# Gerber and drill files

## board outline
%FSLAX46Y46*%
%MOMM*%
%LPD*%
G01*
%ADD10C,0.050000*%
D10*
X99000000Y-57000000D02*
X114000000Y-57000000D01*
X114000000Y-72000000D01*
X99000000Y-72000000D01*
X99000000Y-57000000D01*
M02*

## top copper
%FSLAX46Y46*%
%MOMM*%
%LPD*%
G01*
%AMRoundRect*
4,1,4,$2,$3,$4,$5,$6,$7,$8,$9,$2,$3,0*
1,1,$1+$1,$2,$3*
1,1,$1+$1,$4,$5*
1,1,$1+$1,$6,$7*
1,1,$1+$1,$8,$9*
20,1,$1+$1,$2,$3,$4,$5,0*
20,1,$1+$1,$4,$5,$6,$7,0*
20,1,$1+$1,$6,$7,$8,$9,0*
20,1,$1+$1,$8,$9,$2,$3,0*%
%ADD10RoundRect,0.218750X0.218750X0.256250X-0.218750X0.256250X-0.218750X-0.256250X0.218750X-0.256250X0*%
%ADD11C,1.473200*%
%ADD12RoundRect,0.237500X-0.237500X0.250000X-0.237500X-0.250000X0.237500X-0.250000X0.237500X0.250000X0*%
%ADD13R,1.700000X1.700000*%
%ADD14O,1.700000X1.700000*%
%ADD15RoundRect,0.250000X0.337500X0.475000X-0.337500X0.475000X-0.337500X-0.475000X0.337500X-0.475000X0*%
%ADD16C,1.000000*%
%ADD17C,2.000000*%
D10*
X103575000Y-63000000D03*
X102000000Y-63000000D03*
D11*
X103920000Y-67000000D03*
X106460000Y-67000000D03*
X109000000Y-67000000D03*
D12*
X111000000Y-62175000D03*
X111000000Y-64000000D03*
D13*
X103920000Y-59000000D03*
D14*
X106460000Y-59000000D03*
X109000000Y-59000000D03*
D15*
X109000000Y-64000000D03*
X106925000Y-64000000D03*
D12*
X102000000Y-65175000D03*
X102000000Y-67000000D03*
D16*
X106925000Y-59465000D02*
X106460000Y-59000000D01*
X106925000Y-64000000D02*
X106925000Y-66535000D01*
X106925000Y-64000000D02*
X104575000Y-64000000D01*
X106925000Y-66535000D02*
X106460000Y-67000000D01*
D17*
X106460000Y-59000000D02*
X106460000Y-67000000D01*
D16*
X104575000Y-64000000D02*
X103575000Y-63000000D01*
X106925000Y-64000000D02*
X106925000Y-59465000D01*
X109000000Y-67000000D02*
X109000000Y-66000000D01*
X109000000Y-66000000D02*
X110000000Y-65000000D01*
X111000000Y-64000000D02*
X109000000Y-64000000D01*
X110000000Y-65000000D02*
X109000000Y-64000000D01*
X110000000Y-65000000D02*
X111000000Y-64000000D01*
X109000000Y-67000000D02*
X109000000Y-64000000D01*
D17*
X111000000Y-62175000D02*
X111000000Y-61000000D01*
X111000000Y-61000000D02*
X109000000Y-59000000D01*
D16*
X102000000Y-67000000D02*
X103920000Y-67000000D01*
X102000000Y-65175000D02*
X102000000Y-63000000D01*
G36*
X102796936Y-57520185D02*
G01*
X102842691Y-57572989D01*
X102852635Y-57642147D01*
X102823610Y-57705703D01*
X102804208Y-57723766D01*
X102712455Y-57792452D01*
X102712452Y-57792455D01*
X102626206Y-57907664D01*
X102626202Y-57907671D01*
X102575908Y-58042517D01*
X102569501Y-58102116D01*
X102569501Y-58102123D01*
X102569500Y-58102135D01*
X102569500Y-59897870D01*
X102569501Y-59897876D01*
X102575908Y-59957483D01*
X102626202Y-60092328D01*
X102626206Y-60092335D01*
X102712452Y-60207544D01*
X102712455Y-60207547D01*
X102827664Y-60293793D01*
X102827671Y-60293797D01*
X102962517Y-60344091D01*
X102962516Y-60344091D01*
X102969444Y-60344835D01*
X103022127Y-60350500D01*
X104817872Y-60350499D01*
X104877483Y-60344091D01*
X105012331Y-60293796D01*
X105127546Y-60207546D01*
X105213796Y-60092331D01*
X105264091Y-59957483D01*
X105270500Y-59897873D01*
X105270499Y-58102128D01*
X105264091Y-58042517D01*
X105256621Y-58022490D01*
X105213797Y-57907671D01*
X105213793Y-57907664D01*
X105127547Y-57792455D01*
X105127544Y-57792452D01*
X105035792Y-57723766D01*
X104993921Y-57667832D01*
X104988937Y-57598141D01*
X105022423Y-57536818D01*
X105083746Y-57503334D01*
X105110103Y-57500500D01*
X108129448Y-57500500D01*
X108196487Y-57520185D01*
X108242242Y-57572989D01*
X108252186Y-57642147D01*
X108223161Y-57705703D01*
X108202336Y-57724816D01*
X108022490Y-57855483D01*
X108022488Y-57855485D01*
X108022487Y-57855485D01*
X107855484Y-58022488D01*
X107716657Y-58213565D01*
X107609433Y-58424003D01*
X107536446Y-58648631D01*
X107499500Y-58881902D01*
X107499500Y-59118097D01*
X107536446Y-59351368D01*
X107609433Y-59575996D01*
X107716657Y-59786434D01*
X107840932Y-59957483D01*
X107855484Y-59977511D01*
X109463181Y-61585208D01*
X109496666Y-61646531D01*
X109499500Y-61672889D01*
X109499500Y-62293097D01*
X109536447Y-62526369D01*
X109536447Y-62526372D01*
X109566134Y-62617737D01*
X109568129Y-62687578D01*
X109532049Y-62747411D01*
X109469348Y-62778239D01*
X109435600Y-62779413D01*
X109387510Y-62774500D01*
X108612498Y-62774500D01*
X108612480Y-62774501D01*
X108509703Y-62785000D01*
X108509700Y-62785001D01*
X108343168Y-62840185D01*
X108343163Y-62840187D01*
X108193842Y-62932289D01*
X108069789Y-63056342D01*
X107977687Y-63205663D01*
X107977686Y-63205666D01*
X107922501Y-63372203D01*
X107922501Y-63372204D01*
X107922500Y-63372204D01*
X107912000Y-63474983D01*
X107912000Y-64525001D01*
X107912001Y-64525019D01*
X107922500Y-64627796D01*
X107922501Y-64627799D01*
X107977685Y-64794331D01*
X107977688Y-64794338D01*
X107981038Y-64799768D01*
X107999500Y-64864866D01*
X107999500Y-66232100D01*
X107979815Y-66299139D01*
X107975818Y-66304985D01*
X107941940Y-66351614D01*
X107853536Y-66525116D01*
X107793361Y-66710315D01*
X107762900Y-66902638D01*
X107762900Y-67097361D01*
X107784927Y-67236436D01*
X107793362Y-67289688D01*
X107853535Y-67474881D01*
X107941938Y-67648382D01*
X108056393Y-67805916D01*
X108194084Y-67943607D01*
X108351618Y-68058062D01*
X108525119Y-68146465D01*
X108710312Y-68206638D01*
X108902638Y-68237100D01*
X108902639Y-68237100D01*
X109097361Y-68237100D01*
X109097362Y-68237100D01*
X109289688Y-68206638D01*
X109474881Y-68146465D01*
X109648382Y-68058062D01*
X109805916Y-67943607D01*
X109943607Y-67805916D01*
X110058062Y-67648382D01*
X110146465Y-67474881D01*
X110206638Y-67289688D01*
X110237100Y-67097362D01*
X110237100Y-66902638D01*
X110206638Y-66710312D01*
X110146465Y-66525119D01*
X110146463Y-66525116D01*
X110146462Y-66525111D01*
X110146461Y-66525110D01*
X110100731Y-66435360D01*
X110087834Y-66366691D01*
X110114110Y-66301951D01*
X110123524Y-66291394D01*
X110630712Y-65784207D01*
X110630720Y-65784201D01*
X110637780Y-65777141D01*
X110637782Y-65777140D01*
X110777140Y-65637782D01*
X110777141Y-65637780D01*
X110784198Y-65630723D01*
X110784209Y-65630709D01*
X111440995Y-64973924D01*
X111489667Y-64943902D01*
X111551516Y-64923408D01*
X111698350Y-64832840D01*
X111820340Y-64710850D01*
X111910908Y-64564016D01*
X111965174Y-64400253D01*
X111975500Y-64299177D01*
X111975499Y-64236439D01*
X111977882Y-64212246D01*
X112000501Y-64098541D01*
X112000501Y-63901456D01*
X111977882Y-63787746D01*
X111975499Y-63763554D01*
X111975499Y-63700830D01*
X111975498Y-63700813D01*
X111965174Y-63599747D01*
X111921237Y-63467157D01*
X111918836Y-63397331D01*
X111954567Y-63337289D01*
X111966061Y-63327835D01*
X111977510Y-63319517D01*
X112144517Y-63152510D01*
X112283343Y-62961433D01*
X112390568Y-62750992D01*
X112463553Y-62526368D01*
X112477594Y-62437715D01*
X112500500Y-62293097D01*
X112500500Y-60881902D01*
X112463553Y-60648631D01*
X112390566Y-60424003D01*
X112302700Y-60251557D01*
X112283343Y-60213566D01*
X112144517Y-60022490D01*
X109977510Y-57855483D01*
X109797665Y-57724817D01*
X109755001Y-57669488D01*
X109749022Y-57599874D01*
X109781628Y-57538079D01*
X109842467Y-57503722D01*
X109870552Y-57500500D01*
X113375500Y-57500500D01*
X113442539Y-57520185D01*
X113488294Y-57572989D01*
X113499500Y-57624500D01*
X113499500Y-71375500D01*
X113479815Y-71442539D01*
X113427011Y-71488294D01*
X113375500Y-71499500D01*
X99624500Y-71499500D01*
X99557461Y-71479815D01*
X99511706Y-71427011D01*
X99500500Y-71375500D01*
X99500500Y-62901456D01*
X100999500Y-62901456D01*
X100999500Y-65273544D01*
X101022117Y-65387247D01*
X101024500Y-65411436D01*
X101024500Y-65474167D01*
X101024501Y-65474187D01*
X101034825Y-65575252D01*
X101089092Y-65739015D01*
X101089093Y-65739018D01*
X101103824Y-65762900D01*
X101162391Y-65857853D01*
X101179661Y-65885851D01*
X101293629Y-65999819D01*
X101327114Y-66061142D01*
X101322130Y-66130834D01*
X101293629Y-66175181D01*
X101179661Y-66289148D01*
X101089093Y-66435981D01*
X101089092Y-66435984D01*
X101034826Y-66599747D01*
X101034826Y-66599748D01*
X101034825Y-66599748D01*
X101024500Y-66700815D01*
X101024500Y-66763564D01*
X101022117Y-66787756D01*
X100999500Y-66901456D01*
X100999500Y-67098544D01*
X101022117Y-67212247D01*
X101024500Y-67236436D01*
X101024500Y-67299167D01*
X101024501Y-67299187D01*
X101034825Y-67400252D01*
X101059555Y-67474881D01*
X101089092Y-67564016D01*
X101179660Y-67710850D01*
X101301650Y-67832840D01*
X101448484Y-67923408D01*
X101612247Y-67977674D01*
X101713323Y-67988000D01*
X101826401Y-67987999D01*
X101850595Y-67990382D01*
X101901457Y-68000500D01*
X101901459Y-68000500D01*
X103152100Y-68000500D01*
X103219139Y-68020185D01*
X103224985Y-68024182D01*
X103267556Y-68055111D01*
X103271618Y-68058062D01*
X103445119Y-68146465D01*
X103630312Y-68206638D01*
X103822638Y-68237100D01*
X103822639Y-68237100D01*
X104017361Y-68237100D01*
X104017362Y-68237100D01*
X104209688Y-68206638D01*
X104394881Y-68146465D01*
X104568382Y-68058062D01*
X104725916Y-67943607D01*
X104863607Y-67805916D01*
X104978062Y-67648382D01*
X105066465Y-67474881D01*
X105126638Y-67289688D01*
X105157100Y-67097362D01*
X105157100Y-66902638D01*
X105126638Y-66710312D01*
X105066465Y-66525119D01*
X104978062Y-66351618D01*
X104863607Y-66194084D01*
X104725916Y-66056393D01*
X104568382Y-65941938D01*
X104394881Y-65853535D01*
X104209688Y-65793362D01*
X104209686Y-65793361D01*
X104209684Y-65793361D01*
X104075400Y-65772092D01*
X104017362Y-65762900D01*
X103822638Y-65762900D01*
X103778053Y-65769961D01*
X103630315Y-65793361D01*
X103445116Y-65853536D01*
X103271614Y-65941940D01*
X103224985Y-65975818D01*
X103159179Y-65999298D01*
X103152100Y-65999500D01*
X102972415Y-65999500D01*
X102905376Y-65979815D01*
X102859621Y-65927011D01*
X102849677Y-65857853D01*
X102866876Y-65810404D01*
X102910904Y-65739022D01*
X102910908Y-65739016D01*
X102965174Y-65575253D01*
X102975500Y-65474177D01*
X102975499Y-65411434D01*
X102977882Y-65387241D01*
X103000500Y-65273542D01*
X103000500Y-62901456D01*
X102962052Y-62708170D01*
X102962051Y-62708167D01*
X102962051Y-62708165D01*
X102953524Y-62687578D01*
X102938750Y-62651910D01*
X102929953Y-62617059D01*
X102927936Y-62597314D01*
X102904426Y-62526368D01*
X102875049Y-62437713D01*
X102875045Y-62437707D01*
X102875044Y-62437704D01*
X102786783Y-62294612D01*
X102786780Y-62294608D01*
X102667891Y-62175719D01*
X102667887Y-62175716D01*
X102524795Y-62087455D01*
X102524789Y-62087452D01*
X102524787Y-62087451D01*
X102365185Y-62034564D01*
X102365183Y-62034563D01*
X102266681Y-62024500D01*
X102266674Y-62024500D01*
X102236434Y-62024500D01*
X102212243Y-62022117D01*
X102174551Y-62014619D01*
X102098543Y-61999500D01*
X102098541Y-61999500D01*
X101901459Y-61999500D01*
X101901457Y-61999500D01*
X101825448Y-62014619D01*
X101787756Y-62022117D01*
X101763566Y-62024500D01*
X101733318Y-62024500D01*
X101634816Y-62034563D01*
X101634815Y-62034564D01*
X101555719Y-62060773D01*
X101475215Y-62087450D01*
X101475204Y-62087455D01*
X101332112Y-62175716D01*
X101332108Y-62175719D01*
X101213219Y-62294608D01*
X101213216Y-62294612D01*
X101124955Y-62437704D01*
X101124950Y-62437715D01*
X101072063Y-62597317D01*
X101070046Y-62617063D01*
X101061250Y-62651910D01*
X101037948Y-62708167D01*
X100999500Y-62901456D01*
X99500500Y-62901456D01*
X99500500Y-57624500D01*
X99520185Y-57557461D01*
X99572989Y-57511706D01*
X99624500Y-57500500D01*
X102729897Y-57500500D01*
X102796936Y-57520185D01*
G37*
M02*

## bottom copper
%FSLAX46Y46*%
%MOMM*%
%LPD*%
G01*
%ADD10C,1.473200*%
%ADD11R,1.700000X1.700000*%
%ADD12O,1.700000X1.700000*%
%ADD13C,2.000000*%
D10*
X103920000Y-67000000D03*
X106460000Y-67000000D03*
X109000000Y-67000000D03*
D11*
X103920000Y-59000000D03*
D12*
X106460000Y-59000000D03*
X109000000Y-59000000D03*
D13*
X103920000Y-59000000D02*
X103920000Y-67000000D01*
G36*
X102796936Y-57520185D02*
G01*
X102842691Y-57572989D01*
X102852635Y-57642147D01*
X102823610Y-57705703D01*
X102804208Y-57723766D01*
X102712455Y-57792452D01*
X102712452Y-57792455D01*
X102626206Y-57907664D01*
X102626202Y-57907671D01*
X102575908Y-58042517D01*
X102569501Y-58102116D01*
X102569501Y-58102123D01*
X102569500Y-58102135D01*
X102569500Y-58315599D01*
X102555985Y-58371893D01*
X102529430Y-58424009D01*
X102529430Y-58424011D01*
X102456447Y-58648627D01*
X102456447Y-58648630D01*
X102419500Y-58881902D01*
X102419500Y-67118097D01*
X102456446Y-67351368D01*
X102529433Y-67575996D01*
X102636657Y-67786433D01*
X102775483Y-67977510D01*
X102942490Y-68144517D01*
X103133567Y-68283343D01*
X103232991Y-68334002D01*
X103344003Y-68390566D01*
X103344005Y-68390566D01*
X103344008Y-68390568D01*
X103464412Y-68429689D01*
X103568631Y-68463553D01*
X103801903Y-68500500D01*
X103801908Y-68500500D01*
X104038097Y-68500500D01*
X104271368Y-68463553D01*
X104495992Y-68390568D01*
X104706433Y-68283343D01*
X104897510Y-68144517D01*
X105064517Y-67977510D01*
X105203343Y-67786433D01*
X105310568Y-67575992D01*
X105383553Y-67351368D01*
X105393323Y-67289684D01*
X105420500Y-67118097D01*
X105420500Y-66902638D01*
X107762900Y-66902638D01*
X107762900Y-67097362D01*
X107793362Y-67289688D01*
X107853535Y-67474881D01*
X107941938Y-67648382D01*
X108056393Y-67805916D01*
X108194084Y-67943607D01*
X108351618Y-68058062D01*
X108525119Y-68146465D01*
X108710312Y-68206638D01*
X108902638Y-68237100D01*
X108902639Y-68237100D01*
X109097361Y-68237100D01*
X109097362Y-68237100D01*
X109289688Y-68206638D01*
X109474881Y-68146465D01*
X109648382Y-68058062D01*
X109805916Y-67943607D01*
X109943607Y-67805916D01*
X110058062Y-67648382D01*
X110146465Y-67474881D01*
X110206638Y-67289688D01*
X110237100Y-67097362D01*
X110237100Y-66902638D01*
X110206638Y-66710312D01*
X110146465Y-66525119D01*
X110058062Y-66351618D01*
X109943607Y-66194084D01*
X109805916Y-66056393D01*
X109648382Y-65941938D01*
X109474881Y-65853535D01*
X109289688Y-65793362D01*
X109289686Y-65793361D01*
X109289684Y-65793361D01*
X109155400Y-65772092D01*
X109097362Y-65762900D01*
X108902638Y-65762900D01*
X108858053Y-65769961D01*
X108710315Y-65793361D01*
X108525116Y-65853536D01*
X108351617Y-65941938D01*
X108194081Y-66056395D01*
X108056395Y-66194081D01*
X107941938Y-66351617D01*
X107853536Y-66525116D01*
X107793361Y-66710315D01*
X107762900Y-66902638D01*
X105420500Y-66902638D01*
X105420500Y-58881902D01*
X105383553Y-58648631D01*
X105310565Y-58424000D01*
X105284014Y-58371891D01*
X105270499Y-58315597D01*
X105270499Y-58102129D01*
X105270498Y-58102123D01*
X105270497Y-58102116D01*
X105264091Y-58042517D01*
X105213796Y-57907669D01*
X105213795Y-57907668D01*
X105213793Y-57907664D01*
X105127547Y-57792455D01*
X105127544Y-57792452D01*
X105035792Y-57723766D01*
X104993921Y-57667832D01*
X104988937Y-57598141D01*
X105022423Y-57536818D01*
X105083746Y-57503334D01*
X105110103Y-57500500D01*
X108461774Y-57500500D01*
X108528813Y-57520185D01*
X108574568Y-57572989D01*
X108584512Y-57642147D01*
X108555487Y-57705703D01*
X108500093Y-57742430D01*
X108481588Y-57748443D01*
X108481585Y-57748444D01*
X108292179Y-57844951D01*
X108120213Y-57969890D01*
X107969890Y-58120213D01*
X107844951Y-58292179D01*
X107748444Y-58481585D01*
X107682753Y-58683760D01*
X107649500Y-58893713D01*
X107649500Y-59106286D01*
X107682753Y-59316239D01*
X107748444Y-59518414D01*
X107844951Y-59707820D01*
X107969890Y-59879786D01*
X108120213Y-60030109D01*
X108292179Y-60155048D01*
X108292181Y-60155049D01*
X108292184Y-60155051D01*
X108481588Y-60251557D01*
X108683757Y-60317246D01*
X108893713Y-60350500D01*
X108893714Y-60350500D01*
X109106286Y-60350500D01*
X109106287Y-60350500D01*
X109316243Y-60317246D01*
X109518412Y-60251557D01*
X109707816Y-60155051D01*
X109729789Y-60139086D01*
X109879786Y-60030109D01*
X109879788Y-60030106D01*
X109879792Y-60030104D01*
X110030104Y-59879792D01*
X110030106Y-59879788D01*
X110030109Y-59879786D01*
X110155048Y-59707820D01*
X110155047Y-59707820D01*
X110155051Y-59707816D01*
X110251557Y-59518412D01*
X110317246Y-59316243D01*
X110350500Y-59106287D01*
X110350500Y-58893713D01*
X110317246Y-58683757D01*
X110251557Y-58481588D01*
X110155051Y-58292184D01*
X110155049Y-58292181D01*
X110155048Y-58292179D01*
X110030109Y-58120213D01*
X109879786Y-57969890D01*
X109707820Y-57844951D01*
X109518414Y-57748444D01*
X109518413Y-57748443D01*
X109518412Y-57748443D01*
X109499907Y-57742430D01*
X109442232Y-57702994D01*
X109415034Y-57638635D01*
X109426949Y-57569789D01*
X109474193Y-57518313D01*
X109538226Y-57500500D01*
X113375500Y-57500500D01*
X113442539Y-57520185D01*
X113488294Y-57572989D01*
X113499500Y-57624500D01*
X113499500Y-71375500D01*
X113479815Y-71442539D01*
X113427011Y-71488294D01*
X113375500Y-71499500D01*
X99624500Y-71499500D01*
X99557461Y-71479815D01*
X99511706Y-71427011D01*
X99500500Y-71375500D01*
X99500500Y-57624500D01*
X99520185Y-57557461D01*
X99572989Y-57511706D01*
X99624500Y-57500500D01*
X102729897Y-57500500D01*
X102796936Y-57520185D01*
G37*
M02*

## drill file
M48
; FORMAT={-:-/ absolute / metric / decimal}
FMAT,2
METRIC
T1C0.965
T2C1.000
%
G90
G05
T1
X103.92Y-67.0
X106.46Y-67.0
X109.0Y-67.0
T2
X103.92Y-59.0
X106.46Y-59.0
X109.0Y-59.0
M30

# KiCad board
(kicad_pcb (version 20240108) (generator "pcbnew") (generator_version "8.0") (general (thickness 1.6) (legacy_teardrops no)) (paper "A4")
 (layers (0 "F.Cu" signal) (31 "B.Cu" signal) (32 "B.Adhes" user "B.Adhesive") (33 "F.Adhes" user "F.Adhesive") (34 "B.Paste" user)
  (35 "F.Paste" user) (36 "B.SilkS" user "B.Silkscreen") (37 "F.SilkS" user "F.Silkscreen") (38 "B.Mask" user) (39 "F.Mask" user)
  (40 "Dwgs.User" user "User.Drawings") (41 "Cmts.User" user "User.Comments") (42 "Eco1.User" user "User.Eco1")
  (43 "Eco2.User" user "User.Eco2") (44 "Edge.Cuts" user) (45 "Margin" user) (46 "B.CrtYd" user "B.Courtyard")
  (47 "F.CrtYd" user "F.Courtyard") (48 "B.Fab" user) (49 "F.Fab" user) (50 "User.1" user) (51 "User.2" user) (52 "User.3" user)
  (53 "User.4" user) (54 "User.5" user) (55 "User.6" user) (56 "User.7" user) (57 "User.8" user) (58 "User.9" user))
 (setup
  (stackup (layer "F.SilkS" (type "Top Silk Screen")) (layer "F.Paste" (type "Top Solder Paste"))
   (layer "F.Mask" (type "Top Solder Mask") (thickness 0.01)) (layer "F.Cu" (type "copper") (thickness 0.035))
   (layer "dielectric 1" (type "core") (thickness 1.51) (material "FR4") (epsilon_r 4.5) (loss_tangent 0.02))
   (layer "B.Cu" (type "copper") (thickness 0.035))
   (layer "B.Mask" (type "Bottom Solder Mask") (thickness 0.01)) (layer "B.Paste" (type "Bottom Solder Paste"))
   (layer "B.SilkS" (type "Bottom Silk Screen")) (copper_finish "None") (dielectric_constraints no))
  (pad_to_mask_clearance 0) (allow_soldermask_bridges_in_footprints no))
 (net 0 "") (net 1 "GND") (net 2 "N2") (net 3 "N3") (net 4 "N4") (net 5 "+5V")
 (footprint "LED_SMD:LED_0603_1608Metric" (layer "F.Cu") (at 102.7875 63 180)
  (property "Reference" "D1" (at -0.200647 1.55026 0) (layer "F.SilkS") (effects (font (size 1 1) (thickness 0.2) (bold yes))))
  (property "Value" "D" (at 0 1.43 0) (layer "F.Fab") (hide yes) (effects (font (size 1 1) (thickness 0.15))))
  (pad "1" smd roundrect (at -0.7875 0 180) (size 0.875 0.95) (layers "F.Cu" "F.Paste" "F.Mask") (roundrect_rratio 0.25) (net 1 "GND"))
  (pad "2" smd roundrect (at 0.7875 0 180) (size 0.875 0.95) (layers "F.Cu" "F.Paste" "F.Mask") (roundrect_rratio 0.25) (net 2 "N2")))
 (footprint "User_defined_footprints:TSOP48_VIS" (layer "F.Cu") (at 103.927304 66.99058)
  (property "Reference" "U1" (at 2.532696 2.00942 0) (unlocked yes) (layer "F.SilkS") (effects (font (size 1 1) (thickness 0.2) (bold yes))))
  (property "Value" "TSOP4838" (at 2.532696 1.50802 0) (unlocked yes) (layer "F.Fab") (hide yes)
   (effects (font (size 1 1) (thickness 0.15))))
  (pad "1" thru_hole circle (at -0.007304 0.00942) (size 1.4732 1.4732) (drill 0.9652) (layers "*.Cu" "*.Mask") (remove_unused_layers no)
   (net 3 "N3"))
  (pad "2" thru_hole circle (at 2.532696 0.00942) (size 1.4732 1.4732) (drill 0.9652) (layers "*.Cu" "*.Mask") (remove_unused_layers no)
   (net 1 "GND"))
  (pad "3" thru_hole circle (at 5.072696 0.00942) (size 1.4732 1.4732) (drill 0.9652) (layers "*.Cu" "*.Mask") (remove_unused_layers no)
   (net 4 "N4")))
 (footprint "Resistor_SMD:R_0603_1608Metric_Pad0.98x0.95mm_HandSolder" (layer "F.Cu") (at 111 63.0875 -90)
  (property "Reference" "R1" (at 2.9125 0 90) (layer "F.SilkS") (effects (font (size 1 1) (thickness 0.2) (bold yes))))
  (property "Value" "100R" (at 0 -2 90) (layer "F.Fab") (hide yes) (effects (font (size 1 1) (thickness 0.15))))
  (pad "1" smd roundrect (at -0.9125 0 270) (size 0.975 0.95) (layers "F.Cu" "F.Paste" "F.Mask") (roundrect_rratio 0.25) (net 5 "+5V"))
  (pad "2" smd roundrect (at 0.9125 0 270) (size 0.975 0.95) (layers "F.Cu" "F.Paste" "F.Mask") (roundrect_rratio 0.25) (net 4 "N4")))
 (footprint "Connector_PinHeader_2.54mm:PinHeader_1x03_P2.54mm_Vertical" (layer "F.Cu") (at 103.92 59 90)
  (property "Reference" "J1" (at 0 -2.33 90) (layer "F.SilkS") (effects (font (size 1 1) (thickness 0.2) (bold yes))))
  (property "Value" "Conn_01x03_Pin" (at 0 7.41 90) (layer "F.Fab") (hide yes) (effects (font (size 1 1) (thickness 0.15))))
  (pad "1" thru_hole rect (at 0 0 90) (size 1.7 1.7) (drill 1) (layers "*.Cu" "*.Mask") (remove_unused_layers no) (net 3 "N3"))
  (pad "2" thru_hole oval (at 0 2.54 90) (size 1.7 1.7) (drill 1) (layers "*.Cu" "*.Mask") (remove_unused_layers no) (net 1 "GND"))
  (pad "3" thru_hole oval (at 0 5.08 90) (size 1.7 1.7) (drill 1) (layers "*.Cu" "*.Mask") (remove_unused_layers no) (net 5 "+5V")))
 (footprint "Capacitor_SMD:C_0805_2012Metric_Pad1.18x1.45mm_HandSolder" (layer "F.Cu") (at 107.9625 64 180)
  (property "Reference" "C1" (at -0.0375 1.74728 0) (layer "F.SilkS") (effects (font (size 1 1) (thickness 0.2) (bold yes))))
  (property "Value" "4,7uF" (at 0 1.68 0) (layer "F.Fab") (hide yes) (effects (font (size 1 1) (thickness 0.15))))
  (pad "1" smd roundrect (at -1.0375 0 180) (size 1.175 1.45) (layers "F.Cu" "F.Paste" "F.Mask") (roundrect_rratio 0.212766) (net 4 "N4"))
  (pad "2" smd roundrect (at 1.0375 0 180) (size 1.175 1.45) (layers "F.Cu" "F.Paste" "F.Mask") (roundrect_rratio 0.212766) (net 1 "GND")))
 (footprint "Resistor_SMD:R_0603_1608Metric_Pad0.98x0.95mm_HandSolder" (layer "F.Cu") (at 102 66.0875 -90)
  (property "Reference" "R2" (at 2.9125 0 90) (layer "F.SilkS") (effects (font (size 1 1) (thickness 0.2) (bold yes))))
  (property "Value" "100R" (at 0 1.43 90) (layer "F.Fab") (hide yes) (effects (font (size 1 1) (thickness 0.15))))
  (pad "1" smd roundrect (at -0.9125 0 270) (size 0.975 0.95) (layers "F.Cu" "F.Paste" "F.Mask") (roundrect_rratio 0.25) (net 2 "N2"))
  (pad "2" smd roundrect (at 0.9125 0 270) (size 0.975 0.95) (layers "F.Cu" "F.Paste" "F.Mask") (roundrect_rratio 0.25) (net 3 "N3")))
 (gr_rect (start 99 57) (end 114 72) (stroke (width 0.05) (type default)) (fill none) (layer "Edge.Cuts"))
 (segment (start 106.925 59.465) (end 106.46 59) (width 1) (layer "F.Cu") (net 1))
 (segment (start 106.925 64) (end 106.925 66.535) (width 1) (layer "F.Cu") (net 1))
 (segment (start 106.925 64) (end 104.575 64) (width 1) (layer "F.Cu") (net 1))
 (segment (start 106.925 66.535) (end 106.46 67) (width 1) (layer "F.Cu") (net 1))
 (segment (start 106.46 59) (end 106.46 67) (width 2) (layer "F.Cu") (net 1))
 (segment (start 104.575 64) (end 103.575 63) (width 1) (layer "F.Cu") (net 1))
 (segment (start 106.925 64) (end 106.925 59.465) (width 1) (layer "F.Cu") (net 1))
 (segment (start 109 67) (end 109 66) (width 1) (layer "F.Cu") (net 4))
 (segment (start 109 66) (end 110 65) (width 1) (layer "F.Cu") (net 4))
 (segment (start 111 64) (end 109 64) (width 1) (layer "F.Cu") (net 4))
 (segment (start 110 65) (end 109 64) (width 1) (layer "F.Cu") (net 4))
 (segment (start 110 65) (end 111 64) (width 1) (layer "F.Cu") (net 4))
 (segment (start 109 67) (end 109 64) (width 1) (layer "F.Cu") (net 4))
 (segment (start 111 62.175) (end 111 61) (width 2) (layer "F.Cu") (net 5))
 (segment (start 111 61) (end 109 59) (width 2) (layer "F.Cu") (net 5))
 (segment (start 102 67) (end 103.92 67) (width 1) (layer "F.Cu") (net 3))
 (segment (start 103.92 59) (end 103.92 67) (width 2) (layer "B.Cu") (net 3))
 (segment (start 102 65.175) (end 102 63) (width 1) (layer "F.Cu") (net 2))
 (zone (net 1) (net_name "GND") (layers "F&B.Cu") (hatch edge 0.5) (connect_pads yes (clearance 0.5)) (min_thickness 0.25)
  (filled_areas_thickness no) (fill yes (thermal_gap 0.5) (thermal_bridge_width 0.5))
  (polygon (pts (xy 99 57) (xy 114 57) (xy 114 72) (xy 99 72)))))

